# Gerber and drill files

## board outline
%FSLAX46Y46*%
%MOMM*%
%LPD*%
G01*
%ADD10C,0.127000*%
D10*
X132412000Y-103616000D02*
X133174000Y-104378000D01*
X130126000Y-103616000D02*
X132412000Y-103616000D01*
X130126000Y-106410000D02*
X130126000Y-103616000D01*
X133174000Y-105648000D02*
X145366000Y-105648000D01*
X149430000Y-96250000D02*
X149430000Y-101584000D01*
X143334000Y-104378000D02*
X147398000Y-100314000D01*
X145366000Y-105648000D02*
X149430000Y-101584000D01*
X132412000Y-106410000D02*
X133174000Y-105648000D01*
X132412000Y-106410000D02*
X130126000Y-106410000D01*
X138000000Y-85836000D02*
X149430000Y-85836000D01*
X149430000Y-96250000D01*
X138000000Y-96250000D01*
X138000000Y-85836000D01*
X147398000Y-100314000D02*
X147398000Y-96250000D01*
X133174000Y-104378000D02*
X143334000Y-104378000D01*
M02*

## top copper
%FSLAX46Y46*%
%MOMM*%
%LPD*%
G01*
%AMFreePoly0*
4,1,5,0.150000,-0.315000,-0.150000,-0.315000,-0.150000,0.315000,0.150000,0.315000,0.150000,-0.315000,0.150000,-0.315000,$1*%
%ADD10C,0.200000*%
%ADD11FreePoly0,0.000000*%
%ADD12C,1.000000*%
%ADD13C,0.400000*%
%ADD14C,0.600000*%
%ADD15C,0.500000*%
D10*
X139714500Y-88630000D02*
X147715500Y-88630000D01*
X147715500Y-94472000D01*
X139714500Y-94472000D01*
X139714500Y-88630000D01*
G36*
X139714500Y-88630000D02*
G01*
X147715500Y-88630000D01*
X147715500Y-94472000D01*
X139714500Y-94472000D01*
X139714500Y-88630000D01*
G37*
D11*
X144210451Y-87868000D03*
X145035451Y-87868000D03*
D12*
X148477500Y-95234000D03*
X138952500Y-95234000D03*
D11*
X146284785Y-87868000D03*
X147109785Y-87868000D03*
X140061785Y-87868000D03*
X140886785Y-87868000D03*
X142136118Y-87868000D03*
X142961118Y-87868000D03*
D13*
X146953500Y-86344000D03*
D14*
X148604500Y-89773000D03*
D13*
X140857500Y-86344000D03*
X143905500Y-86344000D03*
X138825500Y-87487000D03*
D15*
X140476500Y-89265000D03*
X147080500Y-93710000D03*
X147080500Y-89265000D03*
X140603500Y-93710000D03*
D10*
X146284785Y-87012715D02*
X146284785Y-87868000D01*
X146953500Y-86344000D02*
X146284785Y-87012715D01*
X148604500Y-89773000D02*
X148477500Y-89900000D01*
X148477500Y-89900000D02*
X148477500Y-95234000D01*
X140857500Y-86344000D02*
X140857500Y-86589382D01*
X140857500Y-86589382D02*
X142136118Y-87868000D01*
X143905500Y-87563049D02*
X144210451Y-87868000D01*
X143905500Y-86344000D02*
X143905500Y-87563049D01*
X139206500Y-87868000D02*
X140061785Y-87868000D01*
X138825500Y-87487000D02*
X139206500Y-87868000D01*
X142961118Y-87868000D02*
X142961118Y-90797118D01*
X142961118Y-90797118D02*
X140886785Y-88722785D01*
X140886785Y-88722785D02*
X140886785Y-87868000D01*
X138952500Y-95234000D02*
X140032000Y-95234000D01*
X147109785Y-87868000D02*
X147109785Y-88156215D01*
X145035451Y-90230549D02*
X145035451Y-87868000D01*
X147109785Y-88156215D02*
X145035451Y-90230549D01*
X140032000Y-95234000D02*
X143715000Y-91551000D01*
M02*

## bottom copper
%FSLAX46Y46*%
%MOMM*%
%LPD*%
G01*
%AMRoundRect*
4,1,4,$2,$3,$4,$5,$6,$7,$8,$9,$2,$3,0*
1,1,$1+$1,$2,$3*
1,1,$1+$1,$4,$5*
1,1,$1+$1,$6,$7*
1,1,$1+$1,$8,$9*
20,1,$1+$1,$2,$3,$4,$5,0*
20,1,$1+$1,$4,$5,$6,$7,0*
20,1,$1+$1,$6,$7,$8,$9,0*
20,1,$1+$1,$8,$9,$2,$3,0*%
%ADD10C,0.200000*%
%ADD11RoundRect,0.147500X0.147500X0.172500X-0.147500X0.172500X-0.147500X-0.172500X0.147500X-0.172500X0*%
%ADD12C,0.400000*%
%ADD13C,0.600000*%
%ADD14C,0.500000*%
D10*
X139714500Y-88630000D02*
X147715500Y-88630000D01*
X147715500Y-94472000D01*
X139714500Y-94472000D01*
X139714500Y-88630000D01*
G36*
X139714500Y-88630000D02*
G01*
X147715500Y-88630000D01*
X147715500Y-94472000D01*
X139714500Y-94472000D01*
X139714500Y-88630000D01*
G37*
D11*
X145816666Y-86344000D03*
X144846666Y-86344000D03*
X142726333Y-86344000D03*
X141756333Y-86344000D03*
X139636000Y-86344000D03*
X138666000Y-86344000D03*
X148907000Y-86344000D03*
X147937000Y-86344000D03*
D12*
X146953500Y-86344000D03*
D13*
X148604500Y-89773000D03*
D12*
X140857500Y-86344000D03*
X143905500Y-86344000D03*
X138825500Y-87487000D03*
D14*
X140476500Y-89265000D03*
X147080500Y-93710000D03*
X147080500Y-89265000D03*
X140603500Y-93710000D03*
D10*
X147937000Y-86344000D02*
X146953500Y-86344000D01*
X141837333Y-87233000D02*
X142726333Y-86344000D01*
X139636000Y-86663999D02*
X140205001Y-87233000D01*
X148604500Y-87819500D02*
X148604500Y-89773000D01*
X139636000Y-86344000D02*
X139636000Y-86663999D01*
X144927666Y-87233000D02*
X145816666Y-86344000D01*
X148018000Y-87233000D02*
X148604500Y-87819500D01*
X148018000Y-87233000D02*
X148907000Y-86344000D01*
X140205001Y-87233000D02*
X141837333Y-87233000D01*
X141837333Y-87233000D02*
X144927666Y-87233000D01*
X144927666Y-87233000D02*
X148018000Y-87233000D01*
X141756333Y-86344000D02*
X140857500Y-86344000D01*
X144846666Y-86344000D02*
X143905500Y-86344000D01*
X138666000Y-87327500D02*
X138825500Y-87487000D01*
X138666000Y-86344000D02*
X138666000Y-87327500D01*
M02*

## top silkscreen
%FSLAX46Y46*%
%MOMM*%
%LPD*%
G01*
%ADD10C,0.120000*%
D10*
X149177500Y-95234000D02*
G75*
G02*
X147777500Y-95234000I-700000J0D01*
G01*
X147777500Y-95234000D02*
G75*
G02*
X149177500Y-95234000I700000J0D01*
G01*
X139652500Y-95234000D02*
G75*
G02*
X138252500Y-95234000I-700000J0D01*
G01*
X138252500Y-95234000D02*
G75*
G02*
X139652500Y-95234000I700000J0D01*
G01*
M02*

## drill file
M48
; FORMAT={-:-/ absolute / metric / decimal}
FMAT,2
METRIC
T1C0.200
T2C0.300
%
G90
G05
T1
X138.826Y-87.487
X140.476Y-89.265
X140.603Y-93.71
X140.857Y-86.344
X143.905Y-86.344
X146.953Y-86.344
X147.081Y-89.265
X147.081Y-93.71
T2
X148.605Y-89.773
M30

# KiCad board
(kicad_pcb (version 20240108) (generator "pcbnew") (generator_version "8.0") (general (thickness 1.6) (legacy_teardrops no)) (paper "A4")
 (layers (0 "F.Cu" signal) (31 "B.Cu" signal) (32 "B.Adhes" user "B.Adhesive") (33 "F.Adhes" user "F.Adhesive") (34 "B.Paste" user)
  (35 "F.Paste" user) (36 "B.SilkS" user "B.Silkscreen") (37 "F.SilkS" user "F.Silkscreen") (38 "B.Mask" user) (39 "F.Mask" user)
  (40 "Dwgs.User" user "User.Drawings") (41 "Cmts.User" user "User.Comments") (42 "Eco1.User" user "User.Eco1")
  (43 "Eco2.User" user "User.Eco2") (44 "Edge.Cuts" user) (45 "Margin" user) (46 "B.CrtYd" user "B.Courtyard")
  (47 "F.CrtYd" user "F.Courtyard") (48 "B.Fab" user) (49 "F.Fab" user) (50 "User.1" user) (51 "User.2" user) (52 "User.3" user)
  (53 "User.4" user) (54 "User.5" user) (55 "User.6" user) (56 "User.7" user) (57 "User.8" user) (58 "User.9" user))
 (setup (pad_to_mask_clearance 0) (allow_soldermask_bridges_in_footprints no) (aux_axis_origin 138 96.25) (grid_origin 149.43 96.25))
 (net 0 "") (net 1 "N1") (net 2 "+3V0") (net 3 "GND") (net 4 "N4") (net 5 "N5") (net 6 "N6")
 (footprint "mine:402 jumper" (layer "F.Cu") (at 144.935451 87.868)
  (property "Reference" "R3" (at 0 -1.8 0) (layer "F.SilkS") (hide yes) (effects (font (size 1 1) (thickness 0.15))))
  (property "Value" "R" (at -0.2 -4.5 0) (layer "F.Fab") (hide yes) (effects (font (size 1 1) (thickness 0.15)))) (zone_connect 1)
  (pad "1" smd custom (at -0.725 0) (size 0.3 0.63) (layers "F.Cu" "F.Mask") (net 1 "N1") (zone_connect 2) (thermal_bridge_angle 45)
   (options (clearance outline) (anchor rect)) (primitives))
  (pad "2" smd custom (at 0.1 0) (size 0.3 0.63) (layers "F.Cu" "F.Mask") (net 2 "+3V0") (zone_connect 2) (thermal_bridge_angle 45)
   (options (clearance outline) (anchor rect)) (primitives)))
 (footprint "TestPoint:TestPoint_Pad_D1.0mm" (layer "F.Cu") (at 148.4775 95.234)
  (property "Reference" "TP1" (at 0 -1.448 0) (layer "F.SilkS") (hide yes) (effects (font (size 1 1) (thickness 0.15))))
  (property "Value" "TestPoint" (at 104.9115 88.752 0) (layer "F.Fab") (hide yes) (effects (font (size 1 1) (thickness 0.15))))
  (fp_circle (center 0 0) (end 0 0.7) (stroke (width 0.12) (type solid)) (fill none) (layer "F.SilkS"))
  (pad "1" smd circle (at 0 0) (size 1 1) (layers "F.Cu" "F.Mask") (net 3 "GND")))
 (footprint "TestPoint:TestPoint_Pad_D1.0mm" (layer "F.Cu") (at 138.9525 95.234)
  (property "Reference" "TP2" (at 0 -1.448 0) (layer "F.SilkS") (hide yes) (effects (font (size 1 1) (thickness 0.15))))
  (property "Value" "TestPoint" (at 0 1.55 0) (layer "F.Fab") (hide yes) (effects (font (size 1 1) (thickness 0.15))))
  (fp_circle (center 0 0) (end 0 0.7) (stroke (width 0.12) (type solid)) (fill none) (layer "F.SilkS"))
  (pad "1" smd circle (at 0 0) (size 1 1) (layers "F.Cu" "F.Mask") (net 2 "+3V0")))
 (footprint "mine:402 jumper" (layer "F.Cu") (at 147.009785 87.868)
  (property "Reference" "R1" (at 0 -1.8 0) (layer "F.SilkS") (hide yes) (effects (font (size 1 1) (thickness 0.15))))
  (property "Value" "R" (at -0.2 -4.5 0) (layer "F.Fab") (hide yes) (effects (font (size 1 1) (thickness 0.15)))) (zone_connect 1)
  (pad "1" smd custom (at -0.725 0) (size 0.3 0.63) (layers "F.Cu" "F.Mask") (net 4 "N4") (zone_connect 2) (thermal_bridge_angle 45)
   (options (clearance outline) (anchor rect)) (primitives))
  (pad "2" smd custom (at 0.1 0) (size 0.3 0.63) (layers "F.Cu" "F.Mask") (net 2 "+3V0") (zone_connect 2) (thermal_bridge_angle 45)
   (options (clearance outline) (anchor rect)) (primitives)))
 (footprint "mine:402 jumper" (layer "F.Cu") (at 140.786785 87.868)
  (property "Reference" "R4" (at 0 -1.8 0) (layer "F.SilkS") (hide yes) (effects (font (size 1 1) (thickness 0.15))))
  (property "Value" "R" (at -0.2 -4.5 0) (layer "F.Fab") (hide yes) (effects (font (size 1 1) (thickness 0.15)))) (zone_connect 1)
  (pad "1" smd custom (at -0.725 0) (size 0.3 0.63) (layers "F.Cu" "F.Mask") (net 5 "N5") (zone_connect 2) (thermal_bridge_angle 45)
   (options (clearance outline) (anchor rect)) (primitives))
  (pad "2" smd custom (at 0.1 0) (size 0.3 0.63) (layers "F.Cu" "F.Mask") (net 2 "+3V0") (zone_connect 2) (thermal_bridge_angle 45)
   (options (clearance outline) (anchor rect)) (primitives)))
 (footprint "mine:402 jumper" (layer "F.Cu") (at 142.861118 87.868)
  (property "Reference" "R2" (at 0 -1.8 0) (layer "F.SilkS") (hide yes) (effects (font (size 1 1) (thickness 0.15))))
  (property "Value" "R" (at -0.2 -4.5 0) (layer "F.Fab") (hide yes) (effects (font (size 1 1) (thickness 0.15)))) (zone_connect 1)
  (pad "1" smd custom (at -0.725 0) (size 0.3 0.63) (layers "F.Cu" "F.Mask") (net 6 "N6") (zone_connect 2) (thermal_bridge_angle 45)
   (options (clearance outline) (anchor rect)) (primitives))
  (pad "2" smd custom (at 0.1 0) (size 0.3 0.63) (layers "F.Cu" "F.Mask") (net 2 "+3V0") (zone_connect 2) (thermal_bridge_angle 45)
   (options (clearance outline) (anchor rect)) (primitives)))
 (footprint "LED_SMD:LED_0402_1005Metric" (layer "B.Cu") (at 145.331666 86.344 180)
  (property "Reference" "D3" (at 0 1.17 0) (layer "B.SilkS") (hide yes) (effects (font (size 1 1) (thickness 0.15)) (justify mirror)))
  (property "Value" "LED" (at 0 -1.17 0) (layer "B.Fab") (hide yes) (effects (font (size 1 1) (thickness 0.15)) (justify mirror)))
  (pad "1" smd roundrect (at -0.485 0 180) (size 0.59 0.64) (layers "B.Cu" "B.Paste" "B.Mask") (roundrect_rratio 0.25) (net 3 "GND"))
  (pad "2" smd roundrect (at 0.485 0 180) (size 0.59 0.64) (layers "B.Cu" "B.Paste" "B.Mask") (roundrect_rratio 0.25) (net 1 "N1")))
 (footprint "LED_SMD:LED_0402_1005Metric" (layer "B.Cu") (at 142.241333 86.344 180)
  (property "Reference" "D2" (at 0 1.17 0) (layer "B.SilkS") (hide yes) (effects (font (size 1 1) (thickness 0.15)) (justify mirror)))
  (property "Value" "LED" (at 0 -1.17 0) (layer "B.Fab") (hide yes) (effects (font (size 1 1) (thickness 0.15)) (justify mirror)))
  (pad "1" smd roundrect (at -0.485 0 180) (size 0.59 0.64) (layers "B.Cu" "B.Paste" "B.Mask") (roundrect_rratio 0.25) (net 3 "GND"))
  (pad "2" smd roundrect (at 0.485 0 180) (size 0.59 0.64) (layers "B.Cu" "B.Paste" "B.Mask") (roundrect_rratio 0.25) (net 6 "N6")))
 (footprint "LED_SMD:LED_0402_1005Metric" (layer "B.Cu") (at 139.151 86.344 180)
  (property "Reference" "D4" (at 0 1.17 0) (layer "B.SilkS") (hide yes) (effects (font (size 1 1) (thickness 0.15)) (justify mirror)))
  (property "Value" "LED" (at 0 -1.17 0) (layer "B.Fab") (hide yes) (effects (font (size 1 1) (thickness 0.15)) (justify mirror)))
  (pad "1" smd roundrect (at -0.485 0 180) (size 0.59 0.64) (layers "B.Cu" "B.Paste" "B.Mask") (roundrect_rratio 0.25) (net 3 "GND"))
  (pad "2" smd roundrect (at 0.485 0 180) (size 0.59 0.64) (layers "B.Cu" "B.Paste" "B.Mask") (roundrect_rratio 0.25) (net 5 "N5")))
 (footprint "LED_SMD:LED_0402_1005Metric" (layer "B.Cu") (at 148.422 86.344 180)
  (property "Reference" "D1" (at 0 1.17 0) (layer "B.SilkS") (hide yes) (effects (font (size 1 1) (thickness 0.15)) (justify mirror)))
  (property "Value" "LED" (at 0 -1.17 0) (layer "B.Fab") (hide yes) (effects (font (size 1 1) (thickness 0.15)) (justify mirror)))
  (pad "1" smd roundrect (at -0.485 0 180) (size 0.59 0.64) (layers "B.Cu" "B.Paste" "B.Mask") (roundrect_rratio 0.25) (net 3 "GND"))
  (pad "2" smd roundrect (at 0.485 0 180) (size 0.59 0.64) (layers "B.Cu" "B.Paste" "B.Mask") (roundrect_rratio 0.25) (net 4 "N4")))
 (gr_rect (start 139.7145 88.63) (end 147.7155 94.472) (stroke (width 0.2) (type default)) (fill solid) (layer "F.Cu") (net 2))
 (gr_rect (start 139.7145 88.63) (end 147.7155 94.472) (stroke (width 0.2) (type default)) (fill solid) (layer "B.Cu") (net 2))
 (gr_line (start 132.412 103.616) (end 133.174 104.378) (stroke (width 0.127) (type default)) (layer "Edge.Cuts"))
 (gr_line (start 130.126 103.616) (end 132.412 103.616) (stroke (width 0.127) (type default)) (layer "Edge.Cuts"))
 (gr_line (start 130.126 106.41) (end 130.126 103.616) (stroke (width 0.127) (type default)) (layer "Edge.Cuts"))
 (gr_line (start 133.174 105.648) (end 145.366 105.648) (stroke (width 0.127) (type default)) (layer "Edge.Cuts"))
 (gr_line (start 149.43 96.25) (end 149.43 101.584) (stroke (width 0.127) (type default)) (layer "Edge.Cuts"))
 (gr_line (start 143.334 104.378) (end 147.398 100.314) (stroke (width 0.127) (type default)) (layer "Edge.Cuts"))
 (gr_line (start 145.366 105.648) (end 149.43 101.584) (stroke (width 0.127) (type default)) (layer "Edge.Cuts"))
 (gr_line (start 132.412 106.41) (end 133.174 105.648) (stroke (width 0.127) (type default)) (layer "Edge.Cuts"))
 (gr_line (start 132.412 106.41) (end 130.126 106.41) (stroke (width 0.127) (type default)) (layer "Edge.Cuts"))
 (gr_rect (start 138 85.836) (end 149.43 96.25) (stroke (width 0.127) (type default)) (fill none) (layer "Edge.Cuts"))
 (gr_line (start 147.398 100.314) (end 147.398 96.25) (stroke (width 0.127) (type default)) (layer "Edge.Cuts"))
 (gr_line (start 133.174 104.378) (end 143.334 104.378) (stroke (width 0.127) (type default)) (layer "Edge.Cuts"))
 (segment (start 146.284785 87.012715) (end 146.284785 87.868) (width 0.2) (layer "F.Cu") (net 4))
 (segment (start 146.9535 86.344) (end 146.284785 87.012715) (width 0.2) (layer "F.Cu") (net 4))
 (via (at 146.9535 86.344) (size 0.4) (drill 0.2) (layers "F.Cu" "B.Cu") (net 4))
 (segment (start 147.937 86.344) (end 146.9535 86.344) (width 0.2) (layer "B.Cu") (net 4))
 (segment (start 148.6045 89.773) (end 148.4775 89.9) (width 0.2) (layer "F.Cu") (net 3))
 (segment (start 148.4775 89.9) (end 148.4775 95.234) (width 0.2) (layer "F.Cu") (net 3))
 (via (at 148.6045 89.773) (size 0.6) (drill 0.3) (layers "F.Cu" "B.Cu") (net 3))
 (segment (start 141.837333 87.233) (end 142.726333 86.344) (width 0.2) (layer "B.Cu") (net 3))
 (segment (start 139.636 86.663999) (end 140.205001 87.233) (width 0.2) (layer "B.Cu") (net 3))
 (segment (start 148.6045 87.8195) (end 148.6045 89.773) (width 0.2) (layer "B.Cu") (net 3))
 (segment (start 139.636 86.344) (end 139.636 86.663999) (width 0.2) (layer "B.Cu") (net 3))
 (segment (start 144.927666 87.233) (end 145.816666 86.344) (width 0.2) (layer "B.Cu") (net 3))
 (segment (start 148.018 87.233) (end 148.6045 87.8195) (width 0.2) (layer "B.Cu") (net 3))
 (segment (start 148.018 87.233) (end 148.907 86.344) (width 0.2) (layer "B.Cu") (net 3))
 (segment (start 140.205001 87.233) (end 141.837333 87.233) (width 0.2) (layer "B.Cu") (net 3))
 (segment (start 141.837333 87.233) (end 144.927666 87.233) (width 0.2) (layer "B.Cu") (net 3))
 (segment (start 144.927666 87.233) (end 148.018 87.233) (width 0.2) (layer "B.Cu") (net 3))
 (segment (start 140.8575 86.344) (end 140.8575 86.589382) (width 0.2) (layer "F.Cu") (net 6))
 (segment (start 140.8575 86.589382) (end 142.136118 87.868) (width 0.2) (layer "F.Cu") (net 6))
 (via (at 140.8575 86.344) (size 0.4) (drill 0.2) (layers "F.Cu" "B.Cu") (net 6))
 (segment (start 141.756333 86.344) (end 140.8575 86.344) (width 0.2) (layer "B.Cu") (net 6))
 (segment (start 143.9055 87.563049) (end 144.210451 87.868) (width 0.2) (layer "F.Cu") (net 1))
 (segment (start 143.9055 86.344) (end 143.9055 87.563049) (width 0.2) (layer "F.Cu") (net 1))
 (via (at 143.9055 86.344) (size 0.4) (drill 0.2) (layers "F.Cu" "B.Cu") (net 1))
 (segment (start 144.846666 86.344) (end 143.9055 86.344) (width 0.2) (layer "B.Cu") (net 1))
 (segment (start 139.2065 87.868) (end 140.061785 87.868) (width 0.2) (layer "F.Cu") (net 5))
 (segment (start 138.8255 87.487) (end 139.2065 87.868) (width 0.2) (layer "F.Cu") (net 5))
 (via (at 138.8255 87.487) (size 0.4) (drill 0.2) (layers "F.Cu" "B.Cu") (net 5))
 (segment (start 138.666 87.3275) (end 138.8255 87.487) (width 0.2) (layer "B.Cu") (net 5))
 (segment (start 138.666 86.344) (end 138.666 87.3275) (width 0.2) (layer "B.Cu") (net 5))
 (segment (start 142.961118 87.868) (end 142.961118 90.797118) (width 0.2) (layer "F.Cu") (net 2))
 (segment (start 142.961118 90.797118) (end 140.886785 88.722785) (width 0.2) (layer "F.Cu") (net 2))
 (segment (start 140.886785 88.722785) (end 140.886785 87.868) (width 0.2) (layer "F.Cu") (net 2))
 (segment (start 138.9525 95.234) (end 140.032 95.234) (width 0.2) (layer "F.Cu") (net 2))
 (segment (start 147.109785 87.868) (end 147.109785 88.156215) (width 0.2) (layer "F.Cu") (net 2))
 (segment (start 145.035451 90.230549) (end 145.035451 87.868) (width 0.2) (layer "F.Cu") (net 2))
 (segment (start 147.109785 88.156215) (end 145.035451 90.230549) (width 0.2) (layer "F.Cu") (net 2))
 (segment (start 140.032 95.234) (end 143.715 91.551) (width 0.2) (layer "F.Cu") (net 2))
 (via (at 140.4765 89.265) (size 0.5) (drill 0.2) (layers "F.Cu" "B.Cu") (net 2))
 (via (at 147.0805 93.71) (size 0.5) (drill 0.2) (layers "F.Cu" "B.Cu") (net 2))
 (via (at 147.0805 89.265) (size 0.5) (drill 0.2) (layers "F.Cu" "B.Cu") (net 2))
 (via (at 140.6035 93.71) (size 0.5) (drill 0.2) (layers "F.Cu" "B.Cu") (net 2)))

